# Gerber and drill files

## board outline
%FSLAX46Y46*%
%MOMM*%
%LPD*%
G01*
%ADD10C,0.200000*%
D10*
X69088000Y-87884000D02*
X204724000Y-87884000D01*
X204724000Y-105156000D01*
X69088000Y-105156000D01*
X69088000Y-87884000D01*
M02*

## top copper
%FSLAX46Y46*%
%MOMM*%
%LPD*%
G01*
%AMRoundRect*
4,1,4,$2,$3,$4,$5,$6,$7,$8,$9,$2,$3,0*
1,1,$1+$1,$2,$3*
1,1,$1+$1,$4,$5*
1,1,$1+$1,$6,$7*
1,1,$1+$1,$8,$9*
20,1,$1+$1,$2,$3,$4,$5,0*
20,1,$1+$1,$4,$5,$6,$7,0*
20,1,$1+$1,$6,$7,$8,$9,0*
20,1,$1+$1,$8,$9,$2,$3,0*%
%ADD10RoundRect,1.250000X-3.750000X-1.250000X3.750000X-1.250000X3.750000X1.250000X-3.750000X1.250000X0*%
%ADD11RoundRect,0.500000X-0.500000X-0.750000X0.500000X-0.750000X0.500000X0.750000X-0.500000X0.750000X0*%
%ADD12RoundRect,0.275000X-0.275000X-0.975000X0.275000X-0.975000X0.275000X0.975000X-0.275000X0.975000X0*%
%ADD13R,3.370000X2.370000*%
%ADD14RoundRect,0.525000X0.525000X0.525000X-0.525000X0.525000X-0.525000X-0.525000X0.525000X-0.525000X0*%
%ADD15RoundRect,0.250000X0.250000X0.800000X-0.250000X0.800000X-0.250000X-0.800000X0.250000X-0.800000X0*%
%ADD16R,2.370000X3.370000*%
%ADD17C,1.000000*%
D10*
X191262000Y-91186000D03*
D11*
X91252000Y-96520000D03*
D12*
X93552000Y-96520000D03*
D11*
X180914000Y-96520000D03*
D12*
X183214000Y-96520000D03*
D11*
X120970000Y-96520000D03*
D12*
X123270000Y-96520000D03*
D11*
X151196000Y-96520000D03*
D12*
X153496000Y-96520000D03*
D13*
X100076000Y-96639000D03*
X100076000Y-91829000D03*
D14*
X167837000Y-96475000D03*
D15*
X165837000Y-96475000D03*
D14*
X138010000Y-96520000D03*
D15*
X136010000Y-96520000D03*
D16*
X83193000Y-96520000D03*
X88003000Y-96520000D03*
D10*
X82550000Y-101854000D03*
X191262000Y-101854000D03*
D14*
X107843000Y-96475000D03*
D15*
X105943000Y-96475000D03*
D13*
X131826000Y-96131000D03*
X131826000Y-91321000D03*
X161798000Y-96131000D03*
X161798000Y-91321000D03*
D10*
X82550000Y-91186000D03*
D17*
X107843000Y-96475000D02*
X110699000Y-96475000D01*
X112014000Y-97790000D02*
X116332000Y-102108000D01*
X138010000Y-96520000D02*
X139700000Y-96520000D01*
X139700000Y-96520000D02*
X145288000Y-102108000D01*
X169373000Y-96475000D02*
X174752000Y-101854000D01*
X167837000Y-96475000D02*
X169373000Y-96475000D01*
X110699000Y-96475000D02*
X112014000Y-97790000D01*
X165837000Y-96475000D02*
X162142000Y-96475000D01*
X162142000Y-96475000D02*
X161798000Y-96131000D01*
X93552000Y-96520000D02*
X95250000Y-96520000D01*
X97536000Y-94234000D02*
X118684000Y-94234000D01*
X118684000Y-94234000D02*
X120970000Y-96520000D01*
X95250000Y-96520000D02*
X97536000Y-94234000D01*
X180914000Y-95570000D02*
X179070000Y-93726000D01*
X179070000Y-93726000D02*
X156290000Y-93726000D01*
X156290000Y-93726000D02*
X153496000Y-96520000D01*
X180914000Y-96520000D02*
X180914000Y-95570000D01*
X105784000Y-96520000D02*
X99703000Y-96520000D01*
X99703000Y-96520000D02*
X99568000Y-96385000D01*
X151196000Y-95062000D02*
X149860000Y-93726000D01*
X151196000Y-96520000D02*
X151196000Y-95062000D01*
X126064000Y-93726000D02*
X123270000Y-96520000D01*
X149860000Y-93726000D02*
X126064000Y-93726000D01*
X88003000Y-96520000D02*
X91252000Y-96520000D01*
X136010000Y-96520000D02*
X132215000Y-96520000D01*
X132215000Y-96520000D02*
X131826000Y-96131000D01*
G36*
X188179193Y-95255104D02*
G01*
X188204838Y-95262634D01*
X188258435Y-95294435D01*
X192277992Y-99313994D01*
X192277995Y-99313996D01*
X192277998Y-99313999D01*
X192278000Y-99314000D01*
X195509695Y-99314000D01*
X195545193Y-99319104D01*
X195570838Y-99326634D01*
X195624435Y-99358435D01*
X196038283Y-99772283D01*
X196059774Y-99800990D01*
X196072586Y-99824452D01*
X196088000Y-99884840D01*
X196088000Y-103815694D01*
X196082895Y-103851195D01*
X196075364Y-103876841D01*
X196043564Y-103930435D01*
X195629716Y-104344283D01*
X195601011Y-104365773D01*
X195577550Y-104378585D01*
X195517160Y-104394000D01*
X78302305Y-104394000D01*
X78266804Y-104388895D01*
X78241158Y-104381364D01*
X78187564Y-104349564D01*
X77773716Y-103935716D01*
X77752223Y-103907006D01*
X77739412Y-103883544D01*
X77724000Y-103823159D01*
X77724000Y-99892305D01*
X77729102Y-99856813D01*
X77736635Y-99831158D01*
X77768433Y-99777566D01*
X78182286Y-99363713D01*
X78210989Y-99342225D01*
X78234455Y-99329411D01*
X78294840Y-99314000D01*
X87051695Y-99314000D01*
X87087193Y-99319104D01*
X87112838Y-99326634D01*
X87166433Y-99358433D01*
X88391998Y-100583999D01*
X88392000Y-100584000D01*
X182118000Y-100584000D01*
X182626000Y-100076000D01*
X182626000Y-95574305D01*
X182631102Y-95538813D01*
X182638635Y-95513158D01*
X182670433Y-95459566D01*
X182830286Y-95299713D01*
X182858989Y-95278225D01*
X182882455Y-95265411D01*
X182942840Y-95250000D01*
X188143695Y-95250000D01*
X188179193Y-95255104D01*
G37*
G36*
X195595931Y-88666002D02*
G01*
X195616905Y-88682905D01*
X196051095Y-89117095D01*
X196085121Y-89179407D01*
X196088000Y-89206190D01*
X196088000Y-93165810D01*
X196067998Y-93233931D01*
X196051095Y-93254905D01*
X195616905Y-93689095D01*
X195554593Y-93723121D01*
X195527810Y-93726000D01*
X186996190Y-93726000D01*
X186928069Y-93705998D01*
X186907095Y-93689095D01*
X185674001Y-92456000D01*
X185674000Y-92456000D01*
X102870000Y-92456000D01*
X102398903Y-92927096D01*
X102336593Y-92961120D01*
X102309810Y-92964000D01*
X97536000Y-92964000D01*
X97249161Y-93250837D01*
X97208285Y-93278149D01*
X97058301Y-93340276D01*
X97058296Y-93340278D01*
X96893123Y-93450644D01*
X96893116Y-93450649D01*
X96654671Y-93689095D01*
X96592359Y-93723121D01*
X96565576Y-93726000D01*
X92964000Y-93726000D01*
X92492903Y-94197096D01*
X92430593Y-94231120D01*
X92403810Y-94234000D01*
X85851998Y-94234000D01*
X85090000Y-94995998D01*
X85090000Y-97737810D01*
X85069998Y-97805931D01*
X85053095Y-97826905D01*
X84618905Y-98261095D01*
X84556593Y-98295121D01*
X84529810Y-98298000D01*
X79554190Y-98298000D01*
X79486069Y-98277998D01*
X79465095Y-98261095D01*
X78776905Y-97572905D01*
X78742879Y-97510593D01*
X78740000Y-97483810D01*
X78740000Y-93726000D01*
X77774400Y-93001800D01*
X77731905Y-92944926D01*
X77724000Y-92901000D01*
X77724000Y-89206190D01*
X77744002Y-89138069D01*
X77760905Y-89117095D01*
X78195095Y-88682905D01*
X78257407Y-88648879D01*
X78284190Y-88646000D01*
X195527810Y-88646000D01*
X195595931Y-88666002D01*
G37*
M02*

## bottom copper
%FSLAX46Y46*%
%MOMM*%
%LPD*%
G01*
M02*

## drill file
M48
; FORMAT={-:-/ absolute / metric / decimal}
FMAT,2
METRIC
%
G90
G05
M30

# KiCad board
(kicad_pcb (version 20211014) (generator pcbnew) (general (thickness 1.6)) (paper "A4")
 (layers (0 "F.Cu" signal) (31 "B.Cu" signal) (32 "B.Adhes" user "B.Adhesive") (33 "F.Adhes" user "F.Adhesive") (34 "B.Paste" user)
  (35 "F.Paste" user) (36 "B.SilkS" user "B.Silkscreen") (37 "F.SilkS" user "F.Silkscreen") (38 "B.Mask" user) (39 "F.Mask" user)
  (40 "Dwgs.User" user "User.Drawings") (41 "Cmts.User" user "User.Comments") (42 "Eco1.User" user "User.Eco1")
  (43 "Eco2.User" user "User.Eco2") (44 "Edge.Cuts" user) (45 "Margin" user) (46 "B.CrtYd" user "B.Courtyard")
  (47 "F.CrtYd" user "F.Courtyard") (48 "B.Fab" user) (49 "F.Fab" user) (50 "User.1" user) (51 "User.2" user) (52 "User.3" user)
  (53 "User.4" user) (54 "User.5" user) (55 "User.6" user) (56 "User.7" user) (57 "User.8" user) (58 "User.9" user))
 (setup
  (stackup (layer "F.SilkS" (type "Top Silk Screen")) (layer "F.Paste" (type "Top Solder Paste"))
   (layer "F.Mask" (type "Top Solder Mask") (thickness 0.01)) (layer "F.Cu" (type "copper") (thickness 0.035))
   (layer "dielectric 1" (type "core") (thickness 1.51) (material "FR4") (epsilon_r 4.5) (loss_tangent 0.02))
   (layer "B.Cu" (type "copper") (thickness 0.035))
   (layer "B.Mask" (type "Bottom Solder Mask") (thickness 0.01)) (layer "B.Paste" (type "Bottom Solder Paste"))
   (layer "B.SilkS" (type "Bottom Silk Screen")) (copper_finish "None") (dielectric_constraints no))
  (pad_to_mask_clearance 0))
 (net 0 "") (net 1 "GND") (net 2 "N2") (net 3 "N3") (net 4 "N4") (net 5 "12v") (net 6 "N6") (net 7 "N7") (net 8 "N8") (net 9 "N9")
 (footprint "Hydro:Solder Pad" (layer "F.Cu") (at 191.262 91.186)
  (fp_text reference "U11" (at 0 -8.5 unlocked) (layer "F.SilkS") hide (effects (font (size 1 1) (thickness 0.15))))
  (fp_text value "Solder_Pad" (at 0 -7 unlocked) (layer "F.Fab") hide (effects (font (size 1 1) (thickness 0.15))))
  (pad "1" smd roundrect (at 0 0) (size 10 5) (layers "F.Cu" "F.Paste" "F.Mask") (roundrect_rratio 0.25) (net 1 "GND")))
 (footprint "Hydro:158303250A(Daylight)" (layer "F.Cu") (at 92.202 96.52)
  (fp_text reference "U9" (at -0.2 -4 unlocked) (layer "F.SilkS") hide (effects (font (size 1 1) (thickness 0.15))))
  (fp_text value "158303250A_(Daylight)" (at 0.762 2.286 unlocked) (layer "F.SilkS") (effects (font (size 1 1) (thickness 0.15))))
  (pad "1" smd roundrect (at -0.95 0) (size 2 2.5) (layers "F.Cu" "F.Paste" "F.Mask") (roundrect_rratio 0.25) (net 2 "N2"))
  (pad "2" smd roundrect (at 1.35 0) (size 1.1 2.5) (layers "F.Cu" "F.Paste" "F.Mask") (roundrect_rratio 0.25) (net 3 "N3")))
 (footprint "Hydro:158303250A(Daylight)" (layer "F.Cu") (at 181.864 96.52)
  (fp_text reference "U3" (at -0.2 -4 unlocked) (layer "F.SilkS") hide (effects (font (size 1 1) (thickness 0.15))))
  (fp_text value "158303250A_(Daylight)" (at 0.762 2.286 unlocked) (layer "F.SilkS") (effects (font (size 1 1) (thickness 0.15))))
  (pad "1" smd roundrect (at -0.95 0) (size 2 2.5) (layers "F.Cu" "F.Paste" "F.Mask") (roundrect_rratio 0.25) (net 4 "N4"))
  (pad "2" smd roundrect (at 1.35 0) (size 1.1 2.5) (layers "F.Cu" "F.Paste" "F.Mask") (roundrect_rratio 0.25) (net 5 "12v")))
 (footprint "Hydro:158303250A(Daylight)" (layer "F.Cu") (at 121.92 96.52)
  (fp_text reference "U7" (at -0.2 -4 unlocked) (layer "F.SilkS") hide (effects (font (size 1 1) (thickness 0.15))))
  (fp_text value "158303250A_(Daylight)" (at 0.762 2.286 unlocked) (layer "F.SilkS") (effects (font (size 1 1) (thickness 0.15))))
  (pad "1" smd roundrect (at -0.95 0) (size 2 2.5) (layers "F.Cu" "F.Paste" "F.Mask") (roundrect_rratio 0.25) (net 3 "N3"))
  (pad "2" smd roundrect (at 1.35 0) (size 1.1 2.5) (layers "F.Cu" "F.Paste" "F.Mask") (roundrect_rratio 0.25) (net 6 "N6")))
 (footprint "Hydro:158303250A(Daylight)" (layer "F.Cu") (at 152.146 96.52)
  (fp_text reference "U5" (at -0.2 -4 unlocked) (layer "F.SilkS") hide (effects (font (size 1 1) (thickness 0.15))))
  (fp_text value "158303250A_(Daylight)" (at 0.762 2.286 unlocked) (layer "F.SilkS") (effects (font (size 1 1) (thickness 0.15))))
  (pad "1" smd roundrect (at -0.95 0) (size 2 2.5) (layers "F.Cu" "F.Paste" "F.Mask") (roundrect_rratio 0.25) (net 6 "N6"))
  (pad "2" smd roundrect (at 1.35 0) (size 1.1 2.5) (layers "F.Cu" "F.Paste" "F.Mask") (roundrect_rratio 0.25) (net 4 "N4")))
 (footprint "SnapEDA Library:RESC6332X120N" (layer "F.Cu") (at 100.076 94.234 90)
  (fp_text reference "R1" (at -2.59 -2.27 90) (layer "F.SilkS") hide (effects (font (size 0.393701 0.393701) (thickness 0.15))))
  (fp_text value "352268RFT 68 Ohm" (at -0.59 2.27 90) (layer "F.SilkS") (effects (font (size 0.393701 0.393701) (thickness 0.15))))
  (pad "1" smd rect locked (at -2.405 0 90) (size 2.37 3.37) (layers "F.Cu" "F.Paste" "F.Mask") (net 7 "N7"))
  (pad "2" smd rect locked (at 2.405 0 90) (size 2.37 3.37) (layers "F.Cu" "F.Paste" "F.Mask") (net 1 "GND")))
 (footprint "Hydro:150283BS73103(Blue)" (layer "F.Cu") (at 168.937 97.575 180)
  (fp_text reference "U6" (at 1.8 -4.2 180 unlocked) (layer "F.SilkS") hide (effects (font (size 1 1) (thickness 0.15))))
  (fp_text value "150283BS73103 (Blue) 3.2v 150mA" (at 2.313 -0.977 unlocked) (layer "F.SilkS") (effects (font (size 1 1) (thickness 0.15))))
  (pad "1" smd roundrect (at 1.1 1.1 180) (size 2.1 2.1) (layers "F.Cu" "F.Paste" "F.Mask") (roundrect_rratio 0.25) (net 5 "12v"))
  (pad "2" smd roundrect (at 3.1 1.1 180) (size 1 2.1) (layers "F.Cu" "F.Paste" "F.Mask") (roundrect_rratio 0.25) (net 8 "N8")))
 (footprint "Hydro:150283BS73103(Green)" (layer "F.Cu") (at 137.16 96.52 180)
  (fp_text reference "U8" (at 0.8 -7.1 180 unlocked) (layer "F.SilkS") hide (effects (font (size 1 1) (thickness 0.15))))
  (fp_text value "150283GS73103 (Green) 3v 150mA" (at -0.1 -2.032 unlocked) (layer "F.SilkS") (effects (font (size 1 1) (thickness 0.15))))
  (pad "1" smd roundrect (at -0.85 0 180) (size 2.1 2.1) (layers "F.Cu" "F.Paste" "F.Mask") (roundrect_rratio 0.25) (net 5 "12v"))
  (pad "2" smd roundrect (at 1.15 0 180) (size 1 2.1) (layers "F.Cu" "F.Paste" "F.Mask") (roundrect_rratio 0.25) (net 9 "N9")))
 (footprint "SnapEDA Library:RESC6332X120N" (layer "F.Cu") (at 85.598 96.52)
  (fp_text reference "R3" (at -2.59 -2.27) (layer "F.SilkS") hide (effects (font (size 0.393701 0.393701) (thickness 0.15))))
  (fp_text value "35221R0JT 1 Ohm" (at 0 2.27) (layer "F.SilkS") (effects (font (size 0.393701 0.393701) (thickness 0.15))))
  (pad "1" smd rect locked (at -2.405 0) (size 2.37 3.37) (layers "F.Cu" "F.Paste" "F.Mask") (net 1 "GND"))
  (pad "2" smd rect locked (at 2.405 0) (size 2.37 3.37) (layers "F.Cu" "F.Paste" "F.Mask") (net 2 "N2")))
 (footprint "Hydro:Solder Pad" (layer "F.Cu") (at 82.55 101.854)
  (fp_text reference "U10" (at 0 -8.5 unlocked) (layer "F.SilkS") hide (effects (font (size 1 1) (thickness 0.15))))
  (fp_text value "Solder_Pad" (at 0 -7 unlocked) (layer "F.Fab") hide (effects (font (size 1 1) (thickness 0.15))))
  (pad "1" smd roundrect (at 0 0) (size 10 5) (layers "F.Cu" "F.Paste" "F.Mask") (roundrect_rratio 0.25) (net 5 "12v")))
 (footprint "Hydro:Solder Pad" (layer "F.Cu") (at 191.262 101.854)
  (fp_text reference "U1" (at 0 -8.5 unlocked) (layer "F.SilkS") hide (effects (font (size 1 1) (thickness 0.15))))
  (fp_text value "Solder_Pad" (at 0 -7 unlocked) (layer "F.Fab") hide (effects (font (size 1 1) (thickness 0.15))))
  (pad "1" smd roundrect (at 0 0) (size 10 5) (layers "F.Cu" "F.Paste" "F.Mask") (roundrect_rratio 0.25) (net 5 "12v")))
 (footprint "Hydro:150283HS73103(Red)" (layer "F.Cu") (at 108.943 97.575 180)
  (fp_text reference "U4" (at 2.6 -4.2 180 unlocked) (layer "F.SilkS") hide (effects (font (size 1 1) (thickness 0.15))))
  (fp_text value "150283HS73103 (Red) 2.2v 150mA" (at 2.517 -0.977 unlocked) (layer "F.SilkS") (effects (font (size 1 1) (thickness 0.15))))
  (pad "1" smd roundrect (at 1.1 1.1 180) (size 2.1 2.1) (layers "F.Cu" "F.Paste" "F.Mask") (roundrect_rratio 0.25) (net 5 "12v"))
  (pad "2" smd roundrect (at 3 1.1 180) (size 1 2.1) (layers "F.Cu" "F.Paste" "F.Mask") (roundrect_rratio 0.25) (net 7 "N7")))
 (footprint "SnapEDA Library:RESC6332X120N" (layer "F.Cu") (at 131.826 93.726 90)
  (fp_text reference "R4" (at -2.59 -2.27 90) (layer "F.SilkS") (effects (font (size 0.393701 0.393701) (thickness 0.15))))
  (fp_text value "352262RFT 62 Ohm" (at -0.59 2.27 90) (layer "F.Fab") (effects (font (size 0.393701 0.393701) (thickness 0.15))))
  (pad "1" smd rect locked (at -2.405 0 90) (size 2.37 3.37) (layers "F.Cu" "F.Paste" "F.Mask") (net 9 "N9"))
  (pad "2" smd rect locked (at 2.405 0 90) (size 2.37 3.37) (layers "F.Cu" "F.Paste" "F.Mask") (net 1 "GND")))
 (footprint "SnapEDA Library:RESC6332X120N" (layer "F.Cu") (at 161.798 93.726 90)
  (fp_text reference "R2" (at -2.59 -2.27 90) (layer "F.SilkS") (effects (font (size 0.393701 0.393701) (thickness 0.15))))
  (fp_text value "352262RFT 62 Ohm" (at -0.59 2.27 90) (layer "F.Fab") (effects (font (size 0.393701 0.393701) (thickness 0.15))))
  (pad "1" smd rect locked (at -2.405 0 90) (size 2.37 3.37) (layers "F.Cu" "F.Paste" "F.Mask") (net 8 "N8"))
  (pad "2" smd rect locked (at 2.405 0 90) (size 2.37 3.37) (layers "F.Cu" "F.Paste" "F.Mask") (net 1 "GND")))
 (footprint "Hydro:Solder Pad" (layer "F.Cu") (at 82.55 91.186)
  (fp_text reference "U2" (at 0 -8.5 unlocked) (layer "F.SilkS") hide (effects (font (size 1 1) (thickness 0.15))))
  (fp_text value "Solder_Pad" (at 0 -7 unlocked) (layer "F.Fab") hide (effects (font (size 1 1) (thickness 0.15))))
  (pad "1" smd roundrect (at 0 0) (size 10 5) (layers "F.Cu" "F.Paste" "F.Mask") (roundrect_rratio 0.25) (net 1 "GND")))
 (gr_rect (start 69.088 87.884) (end 204.724 105.156) (layer "Edge.Cuts") (width 0.2) (fill none))
 (segment (start 107.843 96.475) (end 110.699 96.475) (width 1) (layer "F.Cu") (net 5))
 (segment (start 112.014 97.79) (end 116.332 102.108) (width 1) (layer "F.Cu") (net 5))
 (segment (start 138.01 96.52) (end 139.7 96.52) (width 1) (layer "F.Cu") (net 5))
 (segment (start 139.7 96.52) (end 145.288 102.108) (width 1) (layer "F.Cu") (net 5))
 (segment (start 169.373 96.475) (end 174.752 101.854) (width 1) (layer "F.Cu") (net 5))
 (segment (start 167.837 96.475) (end 169.373 96.475) (width 1) (layer "F.Cu") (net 5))
 (segment (start 110.699 96.475) (end 112.014 97.79) (width 1) (layer "F.Cu") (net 5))
 (segment (start 165.837 96.475) (end 162.142 96.475) (width 1) (layer "F.Cu") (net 8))
 (segment (start 162.142 96.475) (end 161.798 96.131) (width 1) (layer "F.Cu") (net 8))
 (segment (start 93.552 96.52) (end 95.25 96.52) (width 1) (layer "F.Cu") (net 3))
 (segment (start 97.536 94.234) (end 118.684 94.234) (width 1) (layer "F.Cu") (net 3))
 (segment (start 118.684 94.234) (end 120.97 96.52) (width 1) (layer "F.Cu") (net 3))
 (segment (start 95.25 96.52) (end 97.536 94.234) (width 1) (layer "F.Cu") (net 3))
 (segment (start 180.914 95.57) (end 179.07 93.726) (width 1) (layer "F.Cu") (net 4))
 (segment (start 179.07 93.726) (end 156.29 93.726) (width 1) (layer "F.Cu") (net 4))
 (segment (start 156.29 93.726) (end 153.496 96.52) (width 1) (layer "F.Cu") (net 4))
 (segment (start 180.914 96.52) (end 180.914 95.57) (width 1) (layer "F.Cu") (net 4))
 (segment (start 105.784 96.52) (end 99.703 96.52) (width 1) (layer "F.Cu") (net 7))
 (segment (start 99.703 96.52) (end 99.568 96.385) (width 1) (layer "F.Cu") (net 7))
 (segment (start 151.196 95.062) (end 149.86 93.726) (width 1) (layer "F.Cu") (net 6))
 (segment (start 151.196 96.52) (end 151.196 95.062) (width 1) (layer "F.Cu") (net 6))
 (segment (start 126.064 93.726) (end 123.27 96.52) (width 1) (layer "F.Cu") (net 6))
 (segment (start 149.86 93.726) (end 126.064 93.726) (width 1) (layer "F.Cu") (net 6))
 (segment (start 88.003 96.52) (end 91.252 96.52) (width 1) (layer "F.Cu") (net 2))
 (segment (start 136.01 96.52) (end 132.215 96.52) (width 1) (layer "F.Cu") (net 9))
 (segment (start 132.215 96.52) (end 131.826 96.131) (width 1) (layer "F.Cu") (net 9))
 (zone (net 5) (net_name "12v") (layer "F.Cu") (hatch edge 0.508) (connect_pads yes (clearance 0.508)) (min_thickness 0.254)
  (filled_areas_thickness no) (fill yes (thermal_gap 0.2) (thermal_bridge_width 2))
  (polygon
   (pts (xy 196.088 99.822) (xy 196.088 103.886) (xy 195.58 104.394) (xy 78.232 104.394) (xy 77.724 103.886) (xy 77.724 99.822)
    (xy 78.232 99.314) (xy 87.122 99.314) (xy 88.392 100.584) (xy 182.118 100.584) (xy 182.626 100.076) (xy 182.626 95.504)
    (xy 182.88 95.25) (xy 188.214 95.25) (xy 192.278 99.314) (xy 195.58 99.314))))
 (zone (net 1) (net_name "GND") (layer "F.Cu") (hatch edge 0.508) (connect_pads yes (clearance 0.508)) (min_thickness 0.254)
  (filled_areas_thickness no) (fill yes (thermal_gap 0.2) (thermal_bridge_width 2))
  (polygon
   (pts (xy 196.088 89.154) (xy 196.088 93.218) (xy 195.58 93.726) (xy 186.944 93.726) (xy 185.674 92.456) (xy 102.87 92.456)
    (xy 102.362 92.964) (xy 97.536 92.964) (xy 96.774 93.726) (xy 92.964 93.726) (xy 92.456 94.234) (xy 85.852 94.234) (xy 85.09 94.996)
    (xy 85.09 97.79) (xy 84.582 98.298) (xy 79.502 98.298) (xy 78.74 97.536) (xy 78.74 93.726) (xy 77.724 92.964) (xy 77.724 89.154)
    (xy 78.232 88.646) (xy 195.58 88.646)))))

